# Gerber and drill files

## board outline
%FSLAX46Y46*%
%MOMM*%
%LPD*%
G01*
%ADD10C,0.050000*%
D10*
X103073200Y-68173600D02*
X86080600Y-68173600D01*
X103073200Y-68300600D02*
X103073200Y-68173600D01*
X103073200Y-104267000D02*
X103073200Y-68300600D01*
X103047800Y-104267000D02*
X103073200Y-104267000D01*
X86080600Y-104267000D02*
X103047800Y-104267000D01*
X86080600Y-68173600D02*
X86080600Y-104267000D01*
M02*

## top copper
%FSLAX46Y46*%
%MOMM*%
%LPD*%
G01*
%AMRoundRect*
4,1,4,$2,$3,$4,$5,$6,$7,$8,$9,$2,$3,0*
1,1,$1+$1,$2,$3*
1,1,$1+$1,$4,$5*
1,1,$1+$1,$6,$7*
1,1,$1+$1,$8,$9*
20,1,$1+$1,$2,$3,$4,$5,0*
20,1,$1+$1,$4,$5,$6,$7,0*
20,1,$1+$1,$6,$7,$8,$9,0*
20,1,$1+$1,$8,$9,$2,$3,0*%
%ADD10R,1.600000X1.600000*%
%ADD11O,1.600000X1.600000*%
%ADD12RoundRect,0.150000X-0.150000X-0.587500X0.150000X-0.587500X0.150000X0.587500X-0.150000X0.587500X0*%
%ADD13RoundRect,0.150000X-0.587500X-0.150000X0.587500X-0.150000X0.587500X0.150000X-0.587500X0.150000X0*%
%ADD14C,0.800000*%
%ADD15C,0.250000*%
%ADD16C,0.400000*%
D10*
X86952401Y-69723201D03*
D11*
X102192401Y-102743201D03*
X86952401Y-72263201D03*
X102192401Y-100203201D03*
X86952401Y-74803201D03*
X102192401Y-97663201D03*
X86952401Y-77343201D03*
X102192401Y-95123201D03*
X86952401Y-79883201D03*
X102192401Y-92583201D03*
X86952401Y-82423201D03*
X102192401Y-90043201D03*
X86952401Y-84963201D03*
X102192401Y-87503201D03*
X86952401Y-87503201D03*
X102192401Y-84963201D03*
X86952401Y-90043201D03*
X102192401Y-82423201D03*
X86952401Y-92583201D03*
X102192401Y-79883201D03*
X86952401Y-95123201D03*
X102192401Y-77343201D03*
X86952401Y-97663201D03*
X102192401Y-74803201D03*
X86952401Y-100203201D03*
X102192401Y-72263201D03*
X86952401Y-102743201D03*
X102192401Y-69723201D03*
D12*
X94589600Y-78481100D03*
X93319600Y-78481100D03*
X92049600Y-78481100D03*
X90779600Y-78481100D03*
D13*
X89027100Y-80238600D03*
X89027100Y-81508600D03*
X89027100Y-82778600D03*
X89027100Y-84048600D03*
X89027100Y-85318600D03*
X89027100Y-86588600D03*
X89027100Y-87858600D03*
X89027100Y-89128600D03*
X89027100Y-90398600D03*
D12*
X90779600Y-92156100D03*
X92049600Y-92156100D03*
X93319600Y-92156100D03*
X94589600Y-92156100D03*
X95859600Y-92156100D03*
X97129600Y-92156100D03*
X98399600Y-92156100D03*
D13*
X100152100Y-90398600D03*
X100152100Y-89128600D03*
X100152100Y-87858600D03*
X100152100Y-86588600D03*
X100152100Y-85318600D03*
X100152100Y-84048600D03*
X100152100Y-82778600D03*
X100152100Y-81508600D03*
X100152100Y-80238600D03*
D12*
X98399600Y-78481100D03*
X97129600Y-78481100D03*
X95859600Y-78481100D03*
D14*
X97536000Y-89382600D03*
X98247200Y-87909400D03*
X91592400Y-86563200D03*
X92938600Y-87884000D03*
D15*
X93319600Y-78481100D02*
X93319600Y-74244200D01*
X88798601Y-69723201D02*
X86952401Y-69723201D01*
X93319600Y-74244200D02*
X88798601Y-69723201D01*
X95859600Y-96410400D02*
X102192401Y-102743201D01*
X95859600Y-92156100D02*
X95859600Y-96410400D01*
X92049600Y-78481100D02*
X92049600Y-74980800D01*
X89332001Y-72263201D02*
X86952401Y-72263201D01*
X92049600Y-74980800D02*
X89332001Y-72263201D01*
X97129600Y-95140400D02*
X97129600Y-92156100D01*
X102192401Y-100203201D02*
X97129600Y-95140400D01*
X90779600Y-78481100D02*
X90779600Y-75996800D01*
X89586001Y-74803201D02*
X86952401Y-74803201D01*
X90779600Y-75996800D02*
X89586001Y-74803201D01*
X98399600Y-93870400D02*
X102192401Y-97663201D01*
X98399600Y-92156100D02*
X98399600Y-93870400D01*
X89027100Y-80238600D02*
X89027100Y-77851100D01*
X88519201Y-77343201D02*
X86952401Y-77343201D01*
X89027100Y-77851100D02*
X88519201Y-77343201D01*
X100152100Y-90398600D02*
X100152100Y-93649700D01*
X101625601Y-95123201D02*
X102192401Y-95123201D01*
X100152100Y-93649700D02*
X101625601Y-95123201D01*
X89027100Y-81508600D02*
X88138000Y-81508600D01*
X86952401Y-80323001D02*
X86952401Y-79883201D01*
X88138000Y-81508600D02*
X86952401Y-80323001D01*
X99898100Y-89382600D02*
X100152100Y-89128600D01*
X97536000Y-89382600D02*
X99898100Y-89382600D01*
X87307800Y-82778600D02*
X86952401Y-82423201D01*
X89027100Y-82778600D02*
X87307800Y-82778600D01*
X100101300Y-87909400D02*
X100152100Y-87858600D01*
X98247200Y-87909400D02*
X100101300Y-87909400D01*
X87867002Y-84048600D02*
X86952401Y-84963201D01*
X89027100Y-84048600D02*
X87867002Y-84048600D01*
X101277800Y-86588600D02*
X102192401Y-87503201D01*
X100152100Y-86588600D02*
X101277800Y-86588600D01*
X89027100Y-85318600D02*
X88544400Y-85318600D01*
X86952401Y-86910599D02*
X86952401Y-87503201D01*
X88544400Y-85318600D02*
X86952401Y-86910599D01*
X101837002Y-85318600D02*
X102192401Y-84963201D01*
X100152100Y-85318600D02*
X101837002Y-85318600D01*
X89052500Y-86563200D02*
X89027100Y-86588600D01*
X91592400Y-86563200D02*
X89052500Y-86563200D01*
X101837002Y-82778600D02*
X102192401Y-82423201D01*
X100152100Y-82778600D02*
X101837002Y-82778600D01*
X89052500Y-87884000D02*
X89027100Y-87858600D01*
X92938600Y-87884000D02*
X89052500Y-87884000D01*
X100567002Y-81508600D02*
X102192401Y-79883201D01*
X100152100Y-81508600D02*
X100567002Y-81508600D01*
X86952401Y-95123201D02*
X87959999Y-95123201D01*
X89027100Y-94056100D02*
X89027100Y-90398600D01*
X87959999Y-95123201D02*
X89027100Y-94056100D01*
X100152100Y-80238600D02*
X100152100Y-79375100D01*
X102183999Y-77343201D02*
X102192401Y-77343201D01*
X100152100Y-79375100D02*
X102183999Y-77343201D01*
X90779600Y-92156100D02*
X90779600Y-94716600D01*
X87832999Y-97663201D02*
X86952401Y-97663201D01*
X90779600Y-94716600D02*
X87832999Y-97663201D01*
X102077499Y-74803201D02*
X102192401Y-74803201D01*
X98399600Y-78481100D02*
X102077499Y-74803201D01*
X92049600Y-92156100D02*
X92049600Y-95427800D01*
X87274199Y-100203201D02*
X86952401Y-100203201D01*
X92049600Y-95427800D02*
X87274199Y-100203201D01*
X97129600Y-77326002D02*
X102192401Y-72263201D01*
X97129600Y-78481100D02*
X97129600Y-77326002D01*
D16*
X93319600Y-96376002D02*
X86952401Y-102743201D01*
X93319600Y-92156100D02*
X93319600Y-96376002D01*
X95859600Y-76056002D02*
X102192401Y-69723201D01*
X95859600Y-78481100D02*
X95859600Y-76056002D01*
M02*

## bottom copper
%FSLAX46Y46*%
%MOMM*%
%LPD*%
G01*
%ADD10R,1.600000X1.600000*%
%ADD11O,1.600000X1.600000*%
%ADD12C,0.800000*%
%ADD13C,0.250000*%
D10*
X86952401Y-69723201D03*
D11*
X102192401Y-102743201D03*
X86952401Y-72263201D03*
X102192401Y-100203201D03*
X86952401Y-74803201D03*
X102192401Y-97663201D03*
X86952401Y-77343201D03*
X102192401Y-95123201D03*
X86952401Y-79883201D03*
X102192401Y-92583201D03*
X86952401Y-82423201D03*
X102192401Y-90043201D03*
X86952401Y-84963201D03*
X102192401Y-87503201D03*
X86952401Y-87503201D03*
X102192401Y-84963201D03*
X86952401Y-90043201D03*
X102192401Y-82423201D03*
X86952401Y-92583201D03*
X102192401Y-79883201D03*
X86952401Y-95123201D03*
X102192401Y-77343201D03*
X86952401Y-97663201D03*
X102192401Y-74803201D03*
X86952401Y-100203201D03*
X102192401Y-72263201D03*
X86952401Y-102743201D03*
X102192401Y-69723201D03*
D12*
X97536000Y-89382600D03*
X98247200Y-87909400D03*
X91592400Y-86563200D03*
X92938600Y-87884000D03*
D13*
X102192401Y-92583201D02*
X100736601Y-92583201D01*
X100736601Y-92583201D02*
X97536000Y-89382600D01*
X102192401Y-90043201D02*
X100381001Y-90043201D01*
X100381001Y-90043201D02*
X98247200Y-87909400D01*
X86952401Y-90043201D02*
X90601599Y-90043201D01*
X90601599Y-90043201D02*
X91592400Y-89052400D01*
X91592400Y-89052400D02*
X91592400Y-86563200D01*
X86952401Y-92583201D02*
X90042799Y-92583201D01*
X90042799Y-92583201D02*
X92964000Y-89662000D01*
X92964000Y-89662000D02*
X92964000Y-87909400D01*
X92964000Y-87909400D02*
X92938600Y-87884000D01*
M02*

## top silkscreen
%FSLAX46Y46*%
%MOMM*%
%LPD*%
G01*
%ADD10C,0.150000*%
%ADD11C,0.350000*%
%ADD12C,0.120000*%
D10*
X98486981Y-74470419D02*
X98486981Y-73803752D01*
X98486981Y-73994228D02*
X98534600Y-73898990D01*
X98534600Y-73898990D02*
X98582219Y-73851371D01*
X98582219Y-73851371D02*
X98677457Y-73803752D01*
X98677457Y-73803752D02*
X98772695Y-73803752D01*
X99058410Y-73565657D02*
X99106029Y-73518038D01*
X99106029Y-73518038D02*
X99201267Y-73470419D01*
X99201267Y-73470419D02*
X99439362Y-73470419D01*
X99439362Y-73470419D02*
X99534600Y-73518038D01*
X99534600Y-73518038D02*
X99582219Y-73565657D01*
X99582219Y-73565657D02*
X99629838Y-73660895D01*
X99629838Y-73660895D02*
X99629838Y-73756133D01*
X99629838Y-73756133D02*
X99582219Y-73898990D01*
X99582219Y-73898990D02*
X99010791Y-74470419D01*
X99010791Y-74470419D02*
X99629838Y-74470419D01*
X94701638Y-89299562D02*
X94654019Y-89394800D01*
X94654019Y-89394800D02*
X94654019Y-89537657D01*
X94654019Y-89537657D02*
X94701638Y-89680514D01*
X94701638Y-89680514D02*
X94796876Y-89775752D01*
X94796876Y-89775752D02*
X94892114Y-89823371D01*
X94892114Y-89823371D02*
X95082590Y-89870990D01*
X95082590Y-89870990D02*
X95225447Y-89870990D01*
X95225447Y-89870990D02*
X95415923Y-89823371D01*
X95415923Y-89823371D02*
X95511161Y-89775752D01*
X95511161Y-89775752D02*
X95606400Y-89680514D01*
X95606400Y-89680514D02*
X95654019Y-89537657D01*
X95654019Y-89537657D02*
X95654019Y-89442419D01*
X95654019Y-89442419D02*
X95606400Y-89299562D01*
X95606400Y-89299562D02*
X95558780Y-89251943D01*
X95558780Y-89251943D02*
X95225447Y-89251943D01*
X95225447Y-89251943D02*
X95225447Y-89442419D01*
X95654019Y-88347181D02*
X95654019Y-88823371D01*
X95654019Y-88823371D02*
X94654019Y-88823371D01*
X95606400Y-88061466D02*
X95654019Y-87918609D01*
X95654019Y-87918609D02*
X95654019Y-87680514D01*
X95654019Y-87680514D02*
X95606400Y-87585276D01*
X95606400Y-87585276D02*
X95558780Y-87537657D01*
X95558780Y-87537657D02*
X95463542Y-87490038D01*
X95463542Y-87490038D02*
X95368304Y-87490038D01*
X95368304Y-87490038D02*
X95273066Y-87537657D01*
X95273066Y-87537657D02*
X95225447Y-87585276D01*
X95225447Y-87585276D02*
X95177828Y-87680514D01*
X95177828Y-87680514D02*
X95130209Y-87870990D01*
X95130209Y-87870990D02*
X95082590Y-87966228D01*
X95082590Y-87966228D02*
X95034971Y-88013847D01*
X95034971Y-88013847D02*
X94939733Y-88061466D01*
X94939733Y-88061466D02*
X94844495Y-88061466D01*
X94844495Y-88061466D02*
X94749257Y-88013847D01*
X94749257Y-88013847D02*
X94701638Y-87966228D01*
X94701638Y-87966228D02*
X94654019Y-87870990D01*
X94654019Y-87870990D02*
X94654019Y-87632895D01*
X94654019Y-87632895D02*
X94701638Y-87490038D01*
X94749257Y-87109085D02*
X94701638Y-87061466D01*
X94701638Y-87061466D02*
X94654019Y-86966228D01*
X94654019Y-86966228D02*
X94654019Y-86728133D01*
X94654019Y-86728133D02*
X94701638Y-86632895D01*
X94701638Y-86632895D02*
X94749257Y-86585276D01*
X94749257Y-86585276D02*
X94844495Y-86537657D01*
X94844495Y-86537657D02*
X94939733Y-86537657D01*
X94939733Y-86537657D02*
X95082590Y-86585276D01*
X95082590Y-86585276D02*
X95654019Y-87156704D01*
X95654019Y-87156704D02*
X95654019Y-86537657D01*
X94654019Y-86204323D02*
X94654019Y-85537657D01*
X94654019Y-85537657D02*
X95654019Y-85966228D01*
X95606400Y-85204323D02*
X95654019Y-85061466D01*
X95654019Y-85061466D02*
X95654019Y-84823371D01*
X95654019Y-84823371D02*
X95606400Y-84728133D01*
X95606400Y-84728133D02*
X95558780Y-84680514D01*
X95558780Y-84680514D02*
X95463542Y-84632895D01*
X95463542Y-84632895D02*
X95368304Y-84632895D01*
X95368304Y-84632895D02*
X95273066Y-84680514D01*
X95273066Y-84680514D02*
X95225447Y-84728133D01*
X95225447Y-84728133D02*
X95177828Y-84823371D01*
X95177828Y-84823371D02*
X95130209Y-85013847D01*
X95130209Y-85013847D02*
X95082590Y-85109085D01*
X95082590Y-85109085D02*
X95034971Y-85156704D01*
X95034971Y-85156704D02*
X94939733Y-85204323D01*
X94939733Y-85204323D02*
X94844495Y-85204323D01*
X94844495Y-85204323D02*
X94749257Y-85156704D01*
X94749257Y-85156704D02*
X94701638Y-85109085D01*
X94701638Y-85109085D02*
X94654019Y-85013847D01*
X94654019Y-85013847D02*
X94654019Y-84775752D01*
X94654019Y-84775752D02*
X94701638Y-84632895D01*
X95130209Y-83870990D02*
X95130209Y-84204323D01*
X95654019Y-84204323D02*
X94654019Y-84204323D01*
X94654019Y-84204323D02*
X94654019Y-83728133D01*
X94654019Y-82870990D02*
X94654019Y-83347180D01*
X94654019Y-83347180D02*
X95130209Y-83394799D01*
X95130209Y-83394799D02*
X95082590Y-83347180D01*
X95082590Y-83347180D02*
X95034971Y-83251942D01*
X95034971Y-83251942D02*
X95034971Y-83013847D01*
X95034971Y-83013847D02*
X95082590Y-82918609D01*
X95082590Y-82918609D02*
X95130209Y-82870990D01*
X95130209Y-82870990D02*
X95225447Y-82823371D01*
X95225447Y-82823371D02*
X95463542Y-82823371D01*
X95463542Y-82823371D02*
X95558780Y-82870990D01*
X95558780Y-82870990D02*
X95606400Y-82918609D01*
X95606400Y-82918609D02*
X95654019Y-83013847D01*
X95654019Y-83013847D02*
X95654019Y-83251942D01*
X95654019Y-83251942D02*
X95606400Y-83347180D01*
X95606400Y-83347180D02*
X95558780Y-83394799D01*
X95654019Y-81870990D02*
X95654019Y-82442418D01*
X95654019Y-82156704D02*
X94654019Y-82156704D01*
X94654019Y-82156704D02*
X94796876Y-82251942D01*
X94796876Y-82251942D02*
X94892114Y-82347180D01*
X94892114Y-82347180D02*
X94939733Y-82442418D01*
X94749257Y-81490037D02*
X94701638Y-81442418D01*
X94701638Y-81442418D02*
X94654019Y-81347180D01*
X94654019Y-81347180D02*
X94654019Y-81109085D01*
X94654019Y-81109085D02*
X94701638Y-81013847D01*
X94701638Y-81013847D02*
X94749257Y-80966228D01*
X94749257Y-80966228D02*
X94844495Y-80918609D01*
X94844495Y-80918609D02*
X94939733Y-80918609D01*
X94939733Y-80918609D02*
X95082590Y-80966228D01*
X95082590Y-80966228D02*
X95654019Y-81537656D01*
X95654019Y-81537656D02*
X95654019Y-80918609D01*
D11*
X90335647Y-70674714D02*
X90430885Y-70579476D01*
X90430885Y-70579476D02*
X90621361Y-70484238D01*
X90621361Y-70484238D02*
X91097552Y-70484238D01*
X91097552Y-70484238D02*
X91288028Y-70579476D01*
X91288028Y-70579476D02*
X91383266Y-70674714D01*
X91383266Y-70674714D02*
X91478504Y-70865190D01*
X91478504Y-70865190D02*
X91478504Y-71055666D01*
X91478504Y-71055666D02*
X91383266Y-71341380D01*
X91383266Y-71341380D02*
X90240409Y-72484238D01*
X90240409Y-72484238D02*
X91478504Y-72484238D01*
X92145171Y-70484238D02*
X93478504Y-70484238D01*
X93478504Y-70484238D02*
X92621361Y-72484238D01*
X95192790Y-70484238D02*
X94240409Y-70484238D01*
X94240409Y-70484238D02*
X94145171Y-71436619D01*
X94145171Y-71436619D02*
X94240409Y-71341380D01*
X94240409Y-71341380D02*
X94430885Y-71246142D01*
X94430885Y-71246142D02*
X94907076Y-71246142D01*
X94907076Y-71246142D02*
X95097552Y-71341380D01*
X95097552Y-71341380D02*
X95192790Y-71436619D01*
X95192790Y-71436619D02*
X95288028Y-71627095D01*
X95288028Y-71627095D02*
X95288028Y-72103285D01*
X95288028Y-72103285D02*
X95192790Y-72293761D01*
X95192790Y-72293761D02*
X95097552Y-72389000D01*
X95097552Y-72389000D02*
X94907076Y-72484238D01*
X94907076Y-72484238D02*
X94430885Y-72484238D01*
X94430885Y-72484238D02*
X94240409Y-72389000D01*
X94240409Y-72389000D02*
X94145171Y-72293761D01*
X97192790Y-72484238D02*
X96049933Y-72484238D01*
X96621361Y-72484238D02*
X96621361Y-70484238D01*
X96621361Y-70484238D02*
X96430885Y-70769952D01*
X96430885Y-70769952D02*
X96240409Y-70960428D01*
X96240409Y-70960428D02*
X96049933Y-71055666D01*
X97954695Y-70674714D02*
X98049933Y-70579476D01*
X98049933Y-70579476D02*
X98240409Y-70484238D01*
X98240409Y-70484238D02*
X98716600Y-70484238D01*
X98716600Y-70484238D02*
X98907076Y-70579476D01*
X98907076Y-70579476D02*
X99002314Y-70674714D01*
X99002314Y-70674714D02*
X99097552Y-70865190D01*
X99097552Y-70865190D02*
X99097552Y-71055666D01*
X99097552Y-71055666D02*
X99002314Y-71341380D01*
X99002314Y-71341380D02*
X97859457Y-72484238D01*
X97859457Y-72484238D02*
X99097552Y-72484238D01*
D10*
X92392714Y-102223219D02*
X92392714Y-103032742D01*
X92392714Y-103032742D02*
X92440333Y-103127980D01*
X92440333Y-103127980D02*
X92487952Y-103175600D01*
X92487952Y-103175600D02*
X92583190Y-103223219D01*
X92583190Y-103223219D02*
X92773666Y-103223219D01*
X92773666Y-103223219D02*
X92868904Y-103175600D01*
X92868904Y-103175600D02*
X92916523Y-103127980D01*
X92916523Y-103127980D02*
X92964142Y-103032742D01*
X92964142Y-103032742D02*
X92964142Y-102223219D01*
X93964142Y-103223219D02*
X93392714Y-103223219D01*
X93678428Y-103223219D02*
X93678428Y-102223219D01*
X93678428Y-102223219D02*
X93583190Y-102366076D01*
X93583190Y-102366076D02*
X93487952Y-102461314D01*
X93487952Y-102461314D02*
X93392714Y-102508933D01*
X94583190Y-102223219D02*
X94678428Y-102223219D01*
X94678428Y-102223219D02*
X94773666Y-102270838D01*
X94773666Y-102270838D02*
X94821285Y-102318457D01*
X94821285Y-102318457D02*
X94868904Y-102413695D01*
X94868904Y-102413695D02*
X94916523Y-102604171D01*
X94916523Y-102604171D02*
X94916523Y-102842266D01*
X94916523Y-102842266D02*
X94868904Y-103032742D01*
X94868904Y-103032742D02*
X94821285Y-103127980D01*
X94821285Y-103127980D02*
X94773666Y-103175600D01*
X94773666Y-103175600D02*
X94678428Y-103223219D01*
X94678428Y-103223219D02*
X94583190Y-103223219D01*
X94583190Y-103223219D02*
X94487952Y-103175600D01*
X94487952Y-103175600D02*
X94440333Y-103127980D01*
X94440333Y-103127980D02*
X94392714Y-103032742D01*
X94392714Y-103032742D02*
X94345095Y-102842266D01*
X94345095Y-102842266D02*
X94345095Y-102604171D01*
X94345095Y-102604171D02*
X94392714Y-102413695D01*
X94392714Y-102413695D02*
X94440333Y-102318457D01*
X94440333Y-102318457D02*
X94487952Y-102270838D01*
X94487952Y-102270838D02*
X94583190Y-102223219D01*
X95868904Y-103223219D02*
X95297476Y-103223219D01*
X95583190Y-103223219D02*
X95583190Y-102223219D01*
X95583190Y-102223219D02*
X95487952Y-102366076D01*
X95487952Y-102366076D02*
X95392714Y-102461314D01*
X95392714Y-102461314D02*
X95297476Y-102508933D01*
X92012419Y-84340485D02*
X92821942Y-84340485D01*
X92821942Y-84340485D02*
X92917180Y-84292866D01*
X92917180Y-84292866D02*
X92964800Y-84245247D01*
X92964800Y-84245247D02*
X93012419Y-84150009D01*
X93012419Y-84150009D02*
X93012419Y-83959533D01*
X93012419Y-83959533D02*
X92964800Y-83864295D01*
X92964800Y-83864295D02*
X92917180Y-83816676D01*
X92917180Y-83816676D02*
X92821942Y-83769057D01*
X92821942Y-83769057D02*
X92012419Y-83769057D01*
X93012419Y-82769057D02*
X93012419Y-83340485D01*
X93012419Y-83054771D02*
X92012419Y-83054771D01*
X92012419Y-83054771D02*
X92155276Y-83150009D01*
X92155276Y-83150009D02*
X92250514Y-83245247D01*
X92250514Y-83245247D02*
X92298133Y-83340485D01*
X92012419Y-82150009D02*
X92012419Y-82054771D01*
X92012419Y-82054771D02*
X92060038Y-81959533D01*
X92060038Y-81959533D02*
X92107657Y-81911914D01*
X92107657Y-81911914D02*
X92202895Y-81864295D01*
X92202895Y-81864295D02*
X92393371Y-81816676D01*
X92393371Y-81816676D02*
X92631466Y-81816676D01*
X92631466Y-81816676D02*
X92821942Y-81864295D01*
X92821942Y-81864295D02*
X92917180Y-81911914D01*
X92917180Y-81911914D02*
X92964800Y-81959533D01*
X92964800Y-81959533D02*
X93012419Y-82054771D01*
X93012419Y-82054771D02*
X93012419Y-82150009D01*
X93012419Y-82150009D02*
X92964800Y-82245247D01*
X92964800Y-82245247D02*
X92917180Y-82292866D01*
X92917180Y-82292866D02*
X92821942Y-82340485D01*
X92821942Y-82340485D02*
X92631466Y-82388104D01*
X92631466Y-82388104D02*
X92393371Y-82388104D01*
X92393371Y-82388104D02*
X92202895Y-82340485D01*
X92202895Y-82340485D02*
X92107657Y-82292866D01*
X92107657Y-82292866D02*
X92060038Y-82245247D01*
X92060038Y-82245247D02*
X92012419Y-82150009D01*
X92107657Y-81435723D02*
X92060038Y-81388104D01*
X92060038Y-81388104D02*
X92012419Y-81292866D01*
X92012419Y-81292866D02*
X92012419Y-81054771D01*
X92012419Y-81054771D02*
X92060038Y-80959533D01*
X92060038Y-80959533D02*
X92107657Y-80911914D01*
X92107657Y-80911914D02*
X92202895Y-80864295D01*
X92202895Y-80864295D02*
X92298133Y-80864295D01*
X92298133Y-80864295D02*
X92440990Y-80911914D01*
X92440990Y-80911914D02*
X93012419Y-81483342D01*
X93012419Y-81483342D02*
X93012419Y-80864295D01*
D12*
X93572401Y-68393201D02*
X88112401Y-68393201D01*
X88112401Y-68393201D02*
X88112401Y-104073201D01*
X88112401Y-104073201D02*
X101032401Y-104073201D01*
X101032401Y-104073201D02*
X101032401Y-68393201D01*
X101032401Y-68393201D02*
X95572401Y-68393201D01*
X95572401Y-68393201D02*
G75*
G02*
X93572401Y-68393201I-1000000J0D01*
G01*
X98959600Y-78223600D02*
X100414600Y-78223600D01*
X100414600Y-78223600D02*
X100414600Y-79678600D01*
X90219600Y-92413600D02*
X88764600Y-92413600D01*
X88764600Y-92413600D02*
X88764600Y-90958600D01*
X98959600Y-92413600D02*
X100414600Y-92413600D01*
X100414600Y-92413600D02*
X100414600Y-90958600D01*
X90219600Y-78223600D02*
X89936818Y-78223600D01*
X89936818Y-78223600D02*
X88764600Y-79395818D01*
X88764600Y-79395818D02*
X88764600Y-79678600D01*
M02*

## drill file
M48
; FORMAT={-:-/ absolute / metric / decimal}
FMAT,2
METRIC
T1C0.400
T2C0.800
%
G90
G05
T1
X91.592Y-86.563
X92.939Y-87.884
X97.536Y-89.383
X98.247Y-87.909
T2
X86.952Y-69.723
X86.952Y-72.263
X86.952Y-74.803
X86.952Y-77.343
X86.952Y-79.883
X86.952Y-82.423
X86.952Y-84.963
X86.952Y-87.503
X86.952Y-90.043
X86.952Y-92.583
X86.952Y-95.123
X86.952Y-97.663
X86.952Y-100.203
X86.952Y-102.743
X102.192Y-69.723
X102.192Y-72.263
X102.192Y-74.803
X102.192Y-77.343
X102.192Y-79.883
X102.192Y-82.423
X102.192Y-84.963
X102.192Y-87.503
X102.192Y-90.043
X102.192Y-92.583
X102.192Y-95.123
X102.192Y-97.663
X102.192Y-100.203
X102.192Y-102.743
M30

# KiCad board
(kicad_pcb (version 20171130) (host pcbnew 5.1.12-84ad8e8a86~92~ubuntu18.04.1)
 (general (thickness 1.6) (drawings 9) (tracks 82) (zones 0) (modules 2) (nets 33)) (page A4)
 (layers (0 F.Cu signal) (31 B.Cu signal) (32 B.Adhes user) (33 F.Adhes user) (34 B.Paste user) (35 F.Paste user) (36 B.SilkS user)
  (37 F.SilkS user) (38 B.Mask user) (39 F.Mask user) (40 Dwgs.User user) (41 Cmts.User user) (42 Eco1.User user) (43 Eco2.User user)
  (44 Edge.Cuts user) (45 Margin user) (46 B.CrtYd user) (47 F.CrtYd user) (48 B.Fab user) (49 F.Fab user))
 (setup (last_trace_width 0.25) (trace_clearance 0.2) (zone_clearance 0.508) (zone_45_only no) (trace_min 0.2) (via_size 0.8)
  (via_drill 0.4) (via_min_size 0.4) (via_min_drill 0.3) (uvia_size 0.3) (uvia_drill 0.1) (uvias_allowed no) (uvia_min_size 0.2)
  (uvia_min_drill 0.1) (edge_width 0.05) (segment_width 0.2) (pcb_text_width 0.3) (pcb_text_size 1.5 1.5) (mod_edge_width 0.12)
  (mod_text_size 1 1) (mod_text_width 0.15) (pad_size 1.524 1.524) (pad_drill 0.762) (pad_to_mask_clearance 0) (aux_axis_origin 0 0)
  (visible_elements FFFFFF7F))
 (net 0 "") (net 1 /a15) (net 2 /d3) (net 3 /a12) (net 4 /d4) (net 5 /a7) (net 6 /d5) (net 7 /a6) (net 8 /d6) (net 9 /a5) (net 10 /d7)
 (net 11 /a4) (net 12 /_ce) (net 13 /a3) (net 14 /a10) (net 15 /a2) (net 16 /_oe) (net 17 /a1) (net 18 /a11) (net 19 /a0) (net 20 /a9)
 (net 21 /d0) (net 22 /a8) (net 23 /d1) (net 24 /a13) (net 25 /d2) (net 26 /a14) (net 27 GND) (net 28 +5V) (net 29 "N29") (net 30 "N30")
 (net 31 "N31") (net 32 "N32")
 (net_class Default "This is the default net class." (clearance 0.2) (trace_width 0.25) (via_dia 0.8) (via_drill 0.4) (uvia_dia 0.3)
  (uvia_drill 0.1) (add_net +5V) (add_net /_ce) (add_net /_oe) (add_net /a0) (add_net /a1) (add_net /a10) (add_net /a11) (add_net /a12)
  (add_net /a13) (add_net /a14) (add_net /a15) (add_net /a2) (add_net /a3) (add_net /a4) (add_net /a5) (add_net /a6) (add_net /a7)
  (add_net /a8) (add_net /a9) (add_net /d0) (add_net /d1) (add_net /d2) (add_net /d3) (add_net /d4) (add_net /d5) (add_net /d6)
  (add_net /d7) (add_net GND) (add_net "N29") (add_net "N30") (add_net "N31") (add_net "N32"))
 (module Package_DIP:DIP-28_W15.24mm (layer F.Cu) (at 86.952401 69.723201)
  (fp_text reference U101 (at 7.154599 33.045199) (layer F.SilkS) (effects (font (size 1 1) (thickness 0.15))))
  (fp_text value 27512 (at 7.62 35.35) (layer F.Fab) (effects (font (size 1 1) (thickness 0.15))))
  (fp_line (start 6.62 -1.33) (end 1.16 -1.33) (layer F.SilkS) (width 0.12))
  (fp_line (start 1.16 -1.33) (end 1.16 34.35) (layer F.SilkS) (width 0.12))
  (fp_line (start 1.16 34.35) (end 14.08 34.35) (layer F.SilkS) (width 0.12))
  (fp_line (start 14.08 34.35) (end 14.08 -1.33) (layer F.SilkS) (width 0.12))
  (fp_line (start 14.08 -1.33) (end 8.62 -1.33) (layer F.SilkS) (width 0.12))
  (fp_arc (start 7.62 -1.33) (end 6.62 -1.33) (angle -180) (layer F.SilkS) (width 0.12))
  (pad 1 thru_hole rect (at 0 0) (size 1.6 1.6) (drill 0.8) (layers *.Cu *.Mask) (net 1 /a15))
  (pad 15 thru_hole oval (at 15.24 33.02) (size 1.6 1.6) (drill 0.8) (layers *.Cu *.Mask) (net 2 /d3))
  (pad 2 thru_hole oval (at 0 2.54) (size 1.6 1.6) (drill 0.8) (layers *.Cu *.Mask) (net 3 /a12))
  (pad 16 thru_hole oval (at 15.24 30.48) (size 1.6 1.6) (drill 0.8) (layers *.Cu *.Mask) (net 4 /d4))
  (pad 3 thru_hole oval (at 0 5.08) (size 1.6 1.6) (drill 0.8) (layers *.Cu *.Mask) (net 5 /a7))
  (pad 17 thru_hole oval (at 15.24 27.94) (size 1.6 1.6) (drill 0.8) (layers *.Cu *.Mask) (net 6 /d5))
  (pad 4 thru_hole oval (at 0 7.62) (size 1.6 1.6) (drill 0.8) (layers *.Cu *.Mask) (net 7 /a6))
  (pad 18 thru_hole oval (at 15.24 25.4) (size 1.6 1.6) (drill 0.8) (layers *.Cu *.Mask) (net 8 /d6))
  (pad 5 thru_hole oval (at 0 10.16) (size 1.6 1.6) (drill 0.8) (layers *.Cu *.Mask) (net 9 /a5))
  (pad 19 thru_hole oval (at 15.24 22.86) (size 1.6 1.6) (drill 0.8) (layers *.Cu *.Mask) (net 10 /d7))
  (pad 6 thru_hole oval (at 0 12.7) (size 1.6 1.6) (drill 0.8) (layers *.Cu *.Mask) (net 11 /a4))
  (pad 20 thru_hole oval (at 15.24 20.32) (size 1.6 1.6) (drill 0.8) (layers *.Cu *.Mask) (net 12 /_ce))
  (pad 7 thru_hole oval (at 0 15.24) (size 1.6 1.6) (drill 0.8) (layers *.Cu *.Mask) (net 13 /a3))
  (pad 21 thru_hole oval (at 15.24 17.78) (size 1.6 1.6) (drill 0.8) (layers *.Cu *.Mask) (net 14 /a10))
  (pad 8 thru_hole oval (at 0 17.78) (size 1.6 1.6) (drill 0.8) (layers *.Cu *.Mask) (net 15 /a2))
  (pad 22 thru_hole oval (at 15.24 15.24) (size 1.6 1.6) (drill 0.8) (layers *.Cu *.Mask) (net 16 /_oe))
  (pad 9 thru_hole oval (at 0 20.32) (size 1.6 1.6) (drill 0.8) (layers *.Cu *.Mask) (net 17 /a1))
  (pad 23 thru_hole oval (at 15.24 12.7) (size 1.6 1.6) (drill 0.8) (layers *.Cu *.Mask) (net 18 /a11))
  (pad 10 thru_hole oval (at 0 22.86) (size 1.6 1.6) (drill 0.8) (layers *.Cu *.Mask) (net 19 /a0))
  (pad 24 thru_hole oval (at 15.24 10.16) (size 1.6 1.6) (drill 0.8) (layers *.Cu *.Mask) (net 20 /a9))
  (pad 11 thru_hole oval (at 0 25.4) (size 1.6 1.6) (drill 0.8) (layers *.Cu *.Mask) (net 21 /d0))
  (pad 25 thru_hole oval (at 15.24 7.62) (size 1.6 1.6) (drill 0.8) (layers *.Cu *.Mask) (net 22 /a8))
  (pad 12 thru_hole oval (at 0 27.94) (size 1.6 1.6) (drill 0.8) (layers *.Cu *.Mask) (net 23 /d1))
  (pad 26 thru_hole oval (at 15.24 5.08) (size 1.6 1.6) (drill 0.8) (layers *.Cu *.Mask) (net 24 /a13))
  (pad 13 thru_hole oval (at 0 30.48) (size 1.6 1.6) (drill 0.8) (layers *.Cu *.Mask) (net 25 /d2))
  (pad 27 thru_hole oval (at 15.24 2.54) (size 1.6 1.6) (drill 0.8) (layers *.Cu *.Mask) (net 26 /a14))
  (pad 14 thru_hole oval (at 0 33.02) (size 1.6 1.6) (drill 0.8) (layers *.Cu *.Mask) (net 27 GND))
  (pad 28 thru_hole oval (at 15.24 0) (size 1.6 1.6) (drill 0.8) (layers *.Cu *.Mask) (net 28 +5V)))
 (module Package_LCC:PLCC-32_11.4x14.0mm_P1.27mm (layer F.Cu) (at 94.5896 85.3186)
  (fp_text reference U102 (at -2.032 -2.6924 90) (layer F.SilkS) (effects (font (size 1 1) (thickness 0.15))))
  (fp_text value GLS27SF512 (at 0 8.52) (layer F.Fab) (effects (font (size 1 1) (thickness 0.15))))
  (fp_line (start 4.37 -7.095) (end 5.825 -7.095) (layer F.SilkS) (width 0.12))
  (fp_line (start 5.825 -7.095) (end 5.825 -5.64) (layer F.SilkS) (width 0.12))
  (fp_line (start -4.37 7.095) (end -5.825 7.095) (layer F.SilkS) (width 0.12))
  (fp_line (start -5.825 7.095) (end -5.825 5.64) (layer F.SilkS) (width 0.12))
  (fp_line (start 4.37 7.095) (end 5.825 7.095) (layer F.SilkS) (width 0.12))
  (fp_line (start 5.825 7.095) (end 5.825 5.64) (layer F.SilkS) (width 0.12))
  (fp_line (start -4.37 -7.095) (end -4.652782 -7.095) (layer F.SilkS) (width 0.12))
  (fp_line (start -4.652782 -7.095) (end -5.825 -5.922782) (layer F.SilkS) (width 0.12))
  (fp_line (start -5.825 -5.922782) (end -5.825 -5.64) (layer F.SilkS) (width 0.12))
  (pad 1 smd roundrect (at 0 -6.8375) (size 0.6 1.475) (layers F.Cu F.Paste F.Mask) (roundrect_rratio 0.25) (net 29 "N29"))
  (pad 2 smd roundrect (at -1.27 -6.8375) (size 0.6 1.475) (layers F.Cu F.Paste F.Mask) (roundrect_rratio 0.25) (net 1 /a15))
  (pad 3 smd roundrect (at -2.54 -6.8375) (size 0.6 1.475) (layers F.Cu F.Paste F.Mask) (roundrect_rratio 0.25) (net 3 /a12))
  (pad 4 smd roundrect (at -3.81 -6.8375) (size 0.6 1.475) (layers F.Cu F.Paste F.Mask) (roundrect_rratio 0.25) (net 5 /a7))
  (pad 5 smd roundrect (at -5.5625 -5.08) (size 1.475 0.6) (layers F.Cu F.Paste F.Mask) (roundrect_rratio 0.25) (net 7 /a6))
  (pad 6 smd roundrect (at -5.5625 -3.81) (size 1.475 0.6) (layers F.Cu F.Paste F.Mask) (roundrect_rratio 0.25) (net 9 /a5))
  (pad 7 smd roundrect (at -5.5625 -2.54) (size 1.475 0.6) (layers F.Cu F.Paste F.Mask) (roundrect_rratio 0.25) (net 11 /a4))
  (pad 8 smd roundrect (at -5.5625 -1.27) (size 1.475 0.6) (layers F.Cu F.Paste F.Mask) (roundrect_rratio 0.25) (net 13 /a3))
  (pad 9 smd roundrect (at -5.5625 0) (size 1.475 0.6) (layers F.Cu F.Paste F.Mask) (roundrect_rratio 0.25) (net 15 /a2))
  (pad 10 smd roundrect (at -5.5625 1.27) (size 1.475 0.6) (layers F.Cu F.Paste F.Mask) (roundrect_rratio 0.25) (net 17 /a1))
  (pad 11 smd roundrect (at -5.5625 2.54) (size 1.475 0.6) (layers F.Cu F.Paste F.Mask) (roundrect_rratio 0.25) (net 19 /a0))
  (pad 12 smd roundrect (at -5.5625 3.81) (size 1.475 0.6) (layers F.Cu F.Paste F.Mask) (roundrect_rratio 0.25) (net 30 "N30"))
  (pad 13 smd roundrect (at -5.5625 5.08) (size 1.475 0.6) (layers F.Cu F.Paste F.Mask) (roundrect_rratio 0.25) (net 21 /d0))
  (pad 14 smd roundrect (at -3.81 6.8375) (size 0.6 1.475) (layers F.Cu F.Paste F.Mask) (roundrect_rratio 0.25) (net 23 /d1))
  (pad 15 smd roundrect (at -2.54 6.8375) (size 0.6 1.475) (layers F.Cu F.Paste F.Mask) (roundrect_rratio 0.25) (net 25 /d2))
  (pad 16 smd roundrect (at -1.27 6.8375) (size 0.6 1.475) (layers F.Cu F.Paste F.Mask) (roundrect_rratio 0.25) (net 27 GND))
  (pad 17 smd roundrect (at 0 6.8375) (size 0.6 1.475) (layers F.Cu F.Paste F.Mask) (roundrect_rratio 0.25) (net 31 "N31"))
  (pad 18 smd roundrect (at 1.27 6.8375) (size 0.6 1.475) (layers F.Cu F.Paste F.Mask) (roundrect_rratio 0.25) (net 2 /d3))
  (pad 19 smd roundrect (at 2.54 6.8375) (size 0.6 1.475) (layers F.Cu F.Paste F.Mask) (roundrect_rratio 0.25) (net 4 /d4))
  (pad 20 smd roundrect (at 3.81 6.8375) (size 0.6 1.475) (layers F.Cu F.Paste F.Mask) (roundrect_rratio 0.25) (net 6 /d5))
  (pad 21 smd roundrect (at 5.5625 5.08) (size 1.475 0.6) (layers F.Cu F.Paste F.Mask) (roundrect_rratio 0.25) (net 8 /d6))
  (pad 22 smd roundrect (at 5.5625 3.81) (size 1.475 0.6) (layers F.Cu F.Paste F.Mask) (roundrect_rratio 0.25) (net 10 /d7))
  (pad 23 smd roundrect (at 5.5625 2.54) (size 1.475 0.6) (layers F.Cu F.Paste F.Mask) (roundrect_rratio 0.25) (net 12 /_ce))
  (pad 24 smd roundrect (at 5.5625 1.27) (size 1.475 0.6) (layers F.Cu F.Paste F.Mask) (roundrect_rratio 0.25) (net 14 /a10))
  (pad 25 smd roundrect (at 5.5625 0) (size 1.475 0.6) (layers F.Cu F.Paste F.Mask) (roundrect_rratio 0.25) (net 16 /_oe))
  (pad 26 smd roundrect (at 5.5625 -1.27) (size 1.475 0.6) (layers F.Cu F.Paste F.Mask) (roundrect_rratio 0.25) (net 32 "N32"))
  (pad 27 smd roundrect (at 5.5625 -2.54) (size 1.475 0.6) (layers F.Cu F.Paste F.Mask) (roundrect_rratio 0.25) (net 18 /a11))
  (pad 28 smd roundrect (at 5.5625 -3.81) (size 1.475 0.6) (layers F.Cu F.Paste F.Mask) (roundrect_rratio 0.25) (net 20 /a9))
  (pad 29 smd roundrect (at 5.5625 -5.08) (size 1.475 0.6) (layers F.Cu F.Paste F.Mask) (roundrect_rratio 0.25) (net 22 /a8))
  (pad 30 smd roundrect (at 3.81 -6.8375) (size 0.6 1.475) (layers F.Cu F.Paste F.Mask) (roundrect_rratio 0.25) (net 24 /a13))
  (pad 31 smd roundrect (at 2.54 -6.8375) (size 0.6 1.475) (layers F.Cu F.Paste F.Mask) (roundrect_rratio 0.25) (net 26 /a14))
  (pad 32 smd roundrect (at 1.27 -6.8375) (size 0.6 1.475) (layers F.Cu F.Paste F.Mask) (roundrect_rratio 0.25) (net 28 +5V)))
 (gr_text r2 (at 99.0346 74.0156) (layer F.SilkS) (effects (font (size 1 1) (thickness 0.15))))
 (gr_line (start 103.0732 68.1736) (end 86.0806 68.1736) (layer Edge.Cuts) (width 0.05))
 (gr_line (start 103.0732 68.3006) (end 103.0732 68.1736) (layer Edge.Cuts) (width 0.05))
 (gr_line (start 103.0732 104.267) (end 103.0732 68.3006) (layer Edge.Cuts) (width 0.05))
 (gr_line (start 103.0478 104.267) (end 103.0732 104.267) (layer Edge.Cuts) (width 0.05))
 (gr_line (start 86.0806 104.267) (end 103.0478 104.267) (layer Edge.Cuts) (width 0.05))
 (gr_line (start 86.0806 68.1736) (end 86.0806 104.267) (layer Edge.Cuts) (width 0.05))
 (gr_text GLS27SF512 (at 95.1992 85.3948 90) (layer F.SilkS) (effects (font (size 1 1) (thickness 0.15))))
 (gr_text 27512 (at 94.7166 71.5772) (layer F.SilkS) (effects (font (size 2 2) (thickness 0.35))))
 (segment (start 93.3196 78.4811) (end 93.3196 74.2442) (width 0.25) (layer F.Cu) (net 1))
 (segment (start 88.798601 69.723201) (end 86.952401 69.723201) (width 0.25) (layer F.Cu) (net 1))
 (segment (start 93.3196 74.2442) (end 88.798601 69.723201) (width 0.25) (layer F.Cu) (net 1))
 (segment (start 95.8596 96.4104) (end 102.192401 102.743201) (width 0.25) (layer F.Cu) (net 2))
 (segment (start 95.8596 92.1561) (end 95.8596 96.4104) (width 0.25) (layer F.Cu) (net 2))
 (segment (start 92.0496 78.4811) (end 92.0496 74.9808) (width 0.25) (layer F.Cu) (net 3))
 (segment (start 89.332001 72.263201) (end 86.952401 72.263201) (width 0.25) (layer F.Cu) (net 3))
 (segment (start 92.0496 74.9808) (end 89.332001 72.263201) (width 0.25) (layer F.Cu) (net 3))
 (segment (start 97.1296 95.1404) (end 97.1296 92.1561) (width 0.25) (layer F.Cu) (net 4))
 (segment (start 102.192401 100.203201) (end 97.1296 95.1404) (width 0.25) (layer F.Cu) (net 4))
 (segment (start 90.7796 78.4811) (end 90.7796 75.9968) (width 0.25) (layer F.Cu) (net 5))
 (segment (start 89.586001 74.803201) (end 86.952401 74.803201) (width 0.25) (layer F.Cu) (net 5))
 (segment (start 90.7796 75.9968) (end 89.586001 74.803201) (width 0.25) (layer F.Cu) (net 5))
 (segment (start 98.3996 93.8704) (end 102.192401 97.663201) (width 0.25) (layer F.Cu) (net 6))
 (segment (start 98.3996 92.1561) (end 98.3996 93.8704) (width 0.25) (layer F.Cu) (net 6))
 (segment (start 89.0271 80.2386) (end 89.0271 77.8511) (width 0.25) (layer F.Cu) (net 7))
 (segment (start 88.519201 77.343201) (end 86.952401 77.343201) (width 0.25) (layer F.Cu) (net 7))
 (segment (start 89.0271 77.8511) (end 88.519201 77.343201) (width 0.25) (layer F.Cu) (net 7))
 (segment (start 100.1521 90.3986) (end 100.1521 93.6497) (width 0.25) (layer F.Cu) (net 8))
 (segment (start 101.625601 95.123201) (end 102.192401 95.123201) (width 0.25) (layer F.Cu) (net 8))
 (segment (start 100.1521 93.6497) (end 101.625601 95.123201) (width 0.25) (layer F.Cu) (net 8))
 (segment (start 89.0271 81.5086) (end 88.138 81.5086) (width 0.25) (layer F.Cu) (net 9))
 (segment (start 86.952401 80.323001) (end 86.952401 79.883201) (width 0.25) (layer F.Cu) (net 9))
 (segment (start 88.138 81.5086) (end 86.952401 80.323001) (width 0.25) (layer F.Cu) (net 9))
 (via (at 97.536 89.3826) (size 0.8) (drill 0.4) (layers F.Cu B.Cu) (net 10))
 (segment (start 102.192401 92.583201) (end 100.736601 92.583201) (width 0.25) (layer B.Cu) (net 10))
 (segment (start 100.736601 92.583201) (end 97.536 89.3826) (width 0.25) (layer B.Cu) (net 10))
 (segment (start 99.8981 89.3826) (end 100.1521 89.1286) (width 0.25) (layer F.Cu) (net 10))
 (segment (start 97.536 89.3826) (end 99.8981 89.3826) (width 0.25) (layer F.Cu) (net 10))
 (segment (start 87.3078 82.7786) (end 86.952401 82.423201) (width 0.25) (layer F.Cu) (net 11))
 (segment (start 89.0271 82.7786) (end 87.3078 82.7786) (width 0.25) (layer F.Cu) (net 11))
 (via (at 98.2472 87.9094) (size 0.8) (drill 0.4) (layers F.Cu B.Cu) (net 12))
 (segment (start 102.192401 90.043201) (end 100.381001 90.043201) (width 0.25) (layer B.Cu) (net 12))
 (segment (start 100.381001 90.043201) (end 98.2472 87.9094) (width 0.25) (layer B.Cu) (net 12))
 (segment (start 100.1013 87.9094) (end 100.1521 87.8586) (width 0.25) (layer F.Cu) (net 12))
 (segment (start 98.2472 87.9094) (end 100.1013 87.9094) (width 0.25) (layer F.Cu) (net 12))
 (segment (start 87.867002 84.0486) (end 86.952401 84.963201) (width 0.25) (layer F.Cu) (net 13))
 (segment (start 89.0271 84.0486) (end 87.867002 84.0486) (width 0.25) (layer F.Cu) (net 13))
 (segment (start 101.2778 86.5886) (end 102.192401 87.503201) (width 0.25) (layer F.Cu) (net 14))
 (segment (start 100.1521 86.5886) (end 101.2778 86.5886) (width 0.25) (layer F.Cu) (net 14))
 (segment (start 89.0271 85.3186) (end 88.5444 85.3186) (width 0.25) (layer F.Cu) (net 15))
 (segment (start 86.952401 86.910599) (end 86.952401 87.503201) (width 0.25) (layer F.Cu) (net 15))
 (segment (start 88.5444 85.3186) (end 86.952401 86.910599) (width 0.25) (layer F.Cu) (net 15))
 (segment (start 101.837002 85.3186) (end 102.192401 84.963201) (width 0.25) (layer F.Cu) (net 16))
 (segment (start 100.1521 85.3186) (end 101.837002 85.3186) (width 0.25) (layer F.Cu) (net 16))
 (segment (start 86.952401 90.043201) (end 90.601599 90.043201) (width 0.25) (layer B.Cu) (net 17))
 (segment (start 90.601599 90.043201) (end 91.5924 89.0524) (width 0.25) (layer B.Cu) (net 17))
 (via (at 91.5924 86.5632) (size 0.8) (drill 0.4) (layers F.Cu B.Cu) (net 17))
 (segment (start 91.5924 89.0524) (end 91.5924 86.5632) (width 0.25) (layer B.Cu) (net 17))
 (segment (start 89.0525 86.5632) (end 89.0271 86.5886) (width 0.25) (layer F.Cu) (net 17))
 (segment (start 91.5924 86.5632) (end 89.0525 86.5632) (width 0.25) (layer F.Cu) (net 17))
 (segment (start 101.837002 82.7786) (end 102.192401 82.423201) (width 0.25) (layer F.Cu) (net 18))
 (segment (start 100.1521 82.7786) (end 101.837002 82.7786) (width 0.25) (layer F.Cu) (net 18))
 (segment (start 86.952401 92.583201) (end 90.042799 92.583201) (width 0.25) (layer B.Cu) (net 19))
 (segment (start 90.042799 92.583201) (end 92.964 89.662) (width 0.25) (layer B.Cu) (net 19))
 (via (at 92.9386 87.884) (size 0.8) (drill 0.4) (layers F.Cu B.Cu) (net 19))
 (segment (start 92.964 89.662) (end 92.964 87.9094) (width 0.25) (layer B.Cu) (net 19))
 (segment (start 92.964 87.9094) (end 92.9386 87.884) (width 0.25) (layer B.Cu) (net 19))
 (segment (start 89.0525 87.884) (end 89.0271 87.8586) (width 0.25) (layer F.Cu) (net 19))
 (segment (start 92.9386 87.884) (end 89.0525 87.884) (width 0.25) (layer F.Cu) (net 19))
 (segment (start 100.567002 81.5086) (end 102.192401 79.883201) (width 0.25) (layer F.Cu) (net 20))
 (segment (start 100.1521 81.5086) (end 100.567002 81.5086) (width 0.25) (layer F.Cu) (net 20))
 (segment (start 86.952401 95.123201) (end 87.959999 95.123201) (width 0.25) (layer F.Cu) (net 21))
 (segment (start 89.0271 94.0561) (end 89.0271 90.3986) (width 0.25) (layer F.Cu) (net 21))
 (segment (start 87.959999 95.123201) (end 89.0271 94.0561) (width 0.25) (layer F.Cu) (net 21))
 (segment (start 100.1521 80.2386) (end 100.1521 79.3751) (width 0.25) (layer F.Cu) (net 22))
 (segment (start 102.183999 77.343201) (end 102.192401 77.343201) (width 0.25) (layer F.Cu) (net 22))
 (segment (start 100.1521 79.3751) (end 102.183999 77.343201) (width 0.25) (layer F.Cu) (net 22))
 (segment (start 90.7796 92.1561) (end 90.7796 94.7166) (width 0.25) (layer F.Cu) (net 23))
 (segment (start 87.832999 97.663201) (end 86.952401 97.663201) (width 0.25) (layer F.Cu) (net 23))
 (segment (start 90.7796 94.7166) (end 87.832999 97.663201) (width 0.25) (layer F.Cu) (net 23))
 (segment (start 102.077499 74.803201) (end 102.192401 74.803201) (width 0.25) (layer F.Cu) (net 24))
 (segment (start 98.3996 78.4811) (end 102.077499 74.803201) (width 0.25) (layer F.Cu) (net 24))
 (segment (start 92.0496 92.1561) (end 92.0496 95.4278) (width 0.25) (layer F.Cu) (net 25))
 (segment (start 87.274199 100.203201) (end 86.952401 100.203201) (width 0.25) (layer F.Cu) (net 25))
 (segment (start 92.0496 95.4278) (end 87.274199 100.203201) (width 0.25) (layer F.Cu) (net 25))
 (segment (start 97.1296 77.326002) (end 102.192401 72.263201) (width 0.25) (layer F.Cu) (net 26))
 (segment (start 97.1296 78.4811) (end 97.1296 77.326002) (width 0.25) (layer F.Cu) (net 26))
 (segment (start 93.3196 96.376002) (end 86.952401 102.743201) (width 0.4) (layer F.Cu) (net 27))
 (segment (start 93.3196 92.1561) (end 93.3196 96.376002) (width 0.4) (layer F.Cu) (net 27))
 (segment (start 95.8596 76.056002) (end 102.192401 69.723201) (width 0.4) (layer F.Cu) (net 28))
 (segment (start 95.8596 78.4811) (end 95.8596 76.056002) (width 0.4) (layer F.Cu) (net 28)))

